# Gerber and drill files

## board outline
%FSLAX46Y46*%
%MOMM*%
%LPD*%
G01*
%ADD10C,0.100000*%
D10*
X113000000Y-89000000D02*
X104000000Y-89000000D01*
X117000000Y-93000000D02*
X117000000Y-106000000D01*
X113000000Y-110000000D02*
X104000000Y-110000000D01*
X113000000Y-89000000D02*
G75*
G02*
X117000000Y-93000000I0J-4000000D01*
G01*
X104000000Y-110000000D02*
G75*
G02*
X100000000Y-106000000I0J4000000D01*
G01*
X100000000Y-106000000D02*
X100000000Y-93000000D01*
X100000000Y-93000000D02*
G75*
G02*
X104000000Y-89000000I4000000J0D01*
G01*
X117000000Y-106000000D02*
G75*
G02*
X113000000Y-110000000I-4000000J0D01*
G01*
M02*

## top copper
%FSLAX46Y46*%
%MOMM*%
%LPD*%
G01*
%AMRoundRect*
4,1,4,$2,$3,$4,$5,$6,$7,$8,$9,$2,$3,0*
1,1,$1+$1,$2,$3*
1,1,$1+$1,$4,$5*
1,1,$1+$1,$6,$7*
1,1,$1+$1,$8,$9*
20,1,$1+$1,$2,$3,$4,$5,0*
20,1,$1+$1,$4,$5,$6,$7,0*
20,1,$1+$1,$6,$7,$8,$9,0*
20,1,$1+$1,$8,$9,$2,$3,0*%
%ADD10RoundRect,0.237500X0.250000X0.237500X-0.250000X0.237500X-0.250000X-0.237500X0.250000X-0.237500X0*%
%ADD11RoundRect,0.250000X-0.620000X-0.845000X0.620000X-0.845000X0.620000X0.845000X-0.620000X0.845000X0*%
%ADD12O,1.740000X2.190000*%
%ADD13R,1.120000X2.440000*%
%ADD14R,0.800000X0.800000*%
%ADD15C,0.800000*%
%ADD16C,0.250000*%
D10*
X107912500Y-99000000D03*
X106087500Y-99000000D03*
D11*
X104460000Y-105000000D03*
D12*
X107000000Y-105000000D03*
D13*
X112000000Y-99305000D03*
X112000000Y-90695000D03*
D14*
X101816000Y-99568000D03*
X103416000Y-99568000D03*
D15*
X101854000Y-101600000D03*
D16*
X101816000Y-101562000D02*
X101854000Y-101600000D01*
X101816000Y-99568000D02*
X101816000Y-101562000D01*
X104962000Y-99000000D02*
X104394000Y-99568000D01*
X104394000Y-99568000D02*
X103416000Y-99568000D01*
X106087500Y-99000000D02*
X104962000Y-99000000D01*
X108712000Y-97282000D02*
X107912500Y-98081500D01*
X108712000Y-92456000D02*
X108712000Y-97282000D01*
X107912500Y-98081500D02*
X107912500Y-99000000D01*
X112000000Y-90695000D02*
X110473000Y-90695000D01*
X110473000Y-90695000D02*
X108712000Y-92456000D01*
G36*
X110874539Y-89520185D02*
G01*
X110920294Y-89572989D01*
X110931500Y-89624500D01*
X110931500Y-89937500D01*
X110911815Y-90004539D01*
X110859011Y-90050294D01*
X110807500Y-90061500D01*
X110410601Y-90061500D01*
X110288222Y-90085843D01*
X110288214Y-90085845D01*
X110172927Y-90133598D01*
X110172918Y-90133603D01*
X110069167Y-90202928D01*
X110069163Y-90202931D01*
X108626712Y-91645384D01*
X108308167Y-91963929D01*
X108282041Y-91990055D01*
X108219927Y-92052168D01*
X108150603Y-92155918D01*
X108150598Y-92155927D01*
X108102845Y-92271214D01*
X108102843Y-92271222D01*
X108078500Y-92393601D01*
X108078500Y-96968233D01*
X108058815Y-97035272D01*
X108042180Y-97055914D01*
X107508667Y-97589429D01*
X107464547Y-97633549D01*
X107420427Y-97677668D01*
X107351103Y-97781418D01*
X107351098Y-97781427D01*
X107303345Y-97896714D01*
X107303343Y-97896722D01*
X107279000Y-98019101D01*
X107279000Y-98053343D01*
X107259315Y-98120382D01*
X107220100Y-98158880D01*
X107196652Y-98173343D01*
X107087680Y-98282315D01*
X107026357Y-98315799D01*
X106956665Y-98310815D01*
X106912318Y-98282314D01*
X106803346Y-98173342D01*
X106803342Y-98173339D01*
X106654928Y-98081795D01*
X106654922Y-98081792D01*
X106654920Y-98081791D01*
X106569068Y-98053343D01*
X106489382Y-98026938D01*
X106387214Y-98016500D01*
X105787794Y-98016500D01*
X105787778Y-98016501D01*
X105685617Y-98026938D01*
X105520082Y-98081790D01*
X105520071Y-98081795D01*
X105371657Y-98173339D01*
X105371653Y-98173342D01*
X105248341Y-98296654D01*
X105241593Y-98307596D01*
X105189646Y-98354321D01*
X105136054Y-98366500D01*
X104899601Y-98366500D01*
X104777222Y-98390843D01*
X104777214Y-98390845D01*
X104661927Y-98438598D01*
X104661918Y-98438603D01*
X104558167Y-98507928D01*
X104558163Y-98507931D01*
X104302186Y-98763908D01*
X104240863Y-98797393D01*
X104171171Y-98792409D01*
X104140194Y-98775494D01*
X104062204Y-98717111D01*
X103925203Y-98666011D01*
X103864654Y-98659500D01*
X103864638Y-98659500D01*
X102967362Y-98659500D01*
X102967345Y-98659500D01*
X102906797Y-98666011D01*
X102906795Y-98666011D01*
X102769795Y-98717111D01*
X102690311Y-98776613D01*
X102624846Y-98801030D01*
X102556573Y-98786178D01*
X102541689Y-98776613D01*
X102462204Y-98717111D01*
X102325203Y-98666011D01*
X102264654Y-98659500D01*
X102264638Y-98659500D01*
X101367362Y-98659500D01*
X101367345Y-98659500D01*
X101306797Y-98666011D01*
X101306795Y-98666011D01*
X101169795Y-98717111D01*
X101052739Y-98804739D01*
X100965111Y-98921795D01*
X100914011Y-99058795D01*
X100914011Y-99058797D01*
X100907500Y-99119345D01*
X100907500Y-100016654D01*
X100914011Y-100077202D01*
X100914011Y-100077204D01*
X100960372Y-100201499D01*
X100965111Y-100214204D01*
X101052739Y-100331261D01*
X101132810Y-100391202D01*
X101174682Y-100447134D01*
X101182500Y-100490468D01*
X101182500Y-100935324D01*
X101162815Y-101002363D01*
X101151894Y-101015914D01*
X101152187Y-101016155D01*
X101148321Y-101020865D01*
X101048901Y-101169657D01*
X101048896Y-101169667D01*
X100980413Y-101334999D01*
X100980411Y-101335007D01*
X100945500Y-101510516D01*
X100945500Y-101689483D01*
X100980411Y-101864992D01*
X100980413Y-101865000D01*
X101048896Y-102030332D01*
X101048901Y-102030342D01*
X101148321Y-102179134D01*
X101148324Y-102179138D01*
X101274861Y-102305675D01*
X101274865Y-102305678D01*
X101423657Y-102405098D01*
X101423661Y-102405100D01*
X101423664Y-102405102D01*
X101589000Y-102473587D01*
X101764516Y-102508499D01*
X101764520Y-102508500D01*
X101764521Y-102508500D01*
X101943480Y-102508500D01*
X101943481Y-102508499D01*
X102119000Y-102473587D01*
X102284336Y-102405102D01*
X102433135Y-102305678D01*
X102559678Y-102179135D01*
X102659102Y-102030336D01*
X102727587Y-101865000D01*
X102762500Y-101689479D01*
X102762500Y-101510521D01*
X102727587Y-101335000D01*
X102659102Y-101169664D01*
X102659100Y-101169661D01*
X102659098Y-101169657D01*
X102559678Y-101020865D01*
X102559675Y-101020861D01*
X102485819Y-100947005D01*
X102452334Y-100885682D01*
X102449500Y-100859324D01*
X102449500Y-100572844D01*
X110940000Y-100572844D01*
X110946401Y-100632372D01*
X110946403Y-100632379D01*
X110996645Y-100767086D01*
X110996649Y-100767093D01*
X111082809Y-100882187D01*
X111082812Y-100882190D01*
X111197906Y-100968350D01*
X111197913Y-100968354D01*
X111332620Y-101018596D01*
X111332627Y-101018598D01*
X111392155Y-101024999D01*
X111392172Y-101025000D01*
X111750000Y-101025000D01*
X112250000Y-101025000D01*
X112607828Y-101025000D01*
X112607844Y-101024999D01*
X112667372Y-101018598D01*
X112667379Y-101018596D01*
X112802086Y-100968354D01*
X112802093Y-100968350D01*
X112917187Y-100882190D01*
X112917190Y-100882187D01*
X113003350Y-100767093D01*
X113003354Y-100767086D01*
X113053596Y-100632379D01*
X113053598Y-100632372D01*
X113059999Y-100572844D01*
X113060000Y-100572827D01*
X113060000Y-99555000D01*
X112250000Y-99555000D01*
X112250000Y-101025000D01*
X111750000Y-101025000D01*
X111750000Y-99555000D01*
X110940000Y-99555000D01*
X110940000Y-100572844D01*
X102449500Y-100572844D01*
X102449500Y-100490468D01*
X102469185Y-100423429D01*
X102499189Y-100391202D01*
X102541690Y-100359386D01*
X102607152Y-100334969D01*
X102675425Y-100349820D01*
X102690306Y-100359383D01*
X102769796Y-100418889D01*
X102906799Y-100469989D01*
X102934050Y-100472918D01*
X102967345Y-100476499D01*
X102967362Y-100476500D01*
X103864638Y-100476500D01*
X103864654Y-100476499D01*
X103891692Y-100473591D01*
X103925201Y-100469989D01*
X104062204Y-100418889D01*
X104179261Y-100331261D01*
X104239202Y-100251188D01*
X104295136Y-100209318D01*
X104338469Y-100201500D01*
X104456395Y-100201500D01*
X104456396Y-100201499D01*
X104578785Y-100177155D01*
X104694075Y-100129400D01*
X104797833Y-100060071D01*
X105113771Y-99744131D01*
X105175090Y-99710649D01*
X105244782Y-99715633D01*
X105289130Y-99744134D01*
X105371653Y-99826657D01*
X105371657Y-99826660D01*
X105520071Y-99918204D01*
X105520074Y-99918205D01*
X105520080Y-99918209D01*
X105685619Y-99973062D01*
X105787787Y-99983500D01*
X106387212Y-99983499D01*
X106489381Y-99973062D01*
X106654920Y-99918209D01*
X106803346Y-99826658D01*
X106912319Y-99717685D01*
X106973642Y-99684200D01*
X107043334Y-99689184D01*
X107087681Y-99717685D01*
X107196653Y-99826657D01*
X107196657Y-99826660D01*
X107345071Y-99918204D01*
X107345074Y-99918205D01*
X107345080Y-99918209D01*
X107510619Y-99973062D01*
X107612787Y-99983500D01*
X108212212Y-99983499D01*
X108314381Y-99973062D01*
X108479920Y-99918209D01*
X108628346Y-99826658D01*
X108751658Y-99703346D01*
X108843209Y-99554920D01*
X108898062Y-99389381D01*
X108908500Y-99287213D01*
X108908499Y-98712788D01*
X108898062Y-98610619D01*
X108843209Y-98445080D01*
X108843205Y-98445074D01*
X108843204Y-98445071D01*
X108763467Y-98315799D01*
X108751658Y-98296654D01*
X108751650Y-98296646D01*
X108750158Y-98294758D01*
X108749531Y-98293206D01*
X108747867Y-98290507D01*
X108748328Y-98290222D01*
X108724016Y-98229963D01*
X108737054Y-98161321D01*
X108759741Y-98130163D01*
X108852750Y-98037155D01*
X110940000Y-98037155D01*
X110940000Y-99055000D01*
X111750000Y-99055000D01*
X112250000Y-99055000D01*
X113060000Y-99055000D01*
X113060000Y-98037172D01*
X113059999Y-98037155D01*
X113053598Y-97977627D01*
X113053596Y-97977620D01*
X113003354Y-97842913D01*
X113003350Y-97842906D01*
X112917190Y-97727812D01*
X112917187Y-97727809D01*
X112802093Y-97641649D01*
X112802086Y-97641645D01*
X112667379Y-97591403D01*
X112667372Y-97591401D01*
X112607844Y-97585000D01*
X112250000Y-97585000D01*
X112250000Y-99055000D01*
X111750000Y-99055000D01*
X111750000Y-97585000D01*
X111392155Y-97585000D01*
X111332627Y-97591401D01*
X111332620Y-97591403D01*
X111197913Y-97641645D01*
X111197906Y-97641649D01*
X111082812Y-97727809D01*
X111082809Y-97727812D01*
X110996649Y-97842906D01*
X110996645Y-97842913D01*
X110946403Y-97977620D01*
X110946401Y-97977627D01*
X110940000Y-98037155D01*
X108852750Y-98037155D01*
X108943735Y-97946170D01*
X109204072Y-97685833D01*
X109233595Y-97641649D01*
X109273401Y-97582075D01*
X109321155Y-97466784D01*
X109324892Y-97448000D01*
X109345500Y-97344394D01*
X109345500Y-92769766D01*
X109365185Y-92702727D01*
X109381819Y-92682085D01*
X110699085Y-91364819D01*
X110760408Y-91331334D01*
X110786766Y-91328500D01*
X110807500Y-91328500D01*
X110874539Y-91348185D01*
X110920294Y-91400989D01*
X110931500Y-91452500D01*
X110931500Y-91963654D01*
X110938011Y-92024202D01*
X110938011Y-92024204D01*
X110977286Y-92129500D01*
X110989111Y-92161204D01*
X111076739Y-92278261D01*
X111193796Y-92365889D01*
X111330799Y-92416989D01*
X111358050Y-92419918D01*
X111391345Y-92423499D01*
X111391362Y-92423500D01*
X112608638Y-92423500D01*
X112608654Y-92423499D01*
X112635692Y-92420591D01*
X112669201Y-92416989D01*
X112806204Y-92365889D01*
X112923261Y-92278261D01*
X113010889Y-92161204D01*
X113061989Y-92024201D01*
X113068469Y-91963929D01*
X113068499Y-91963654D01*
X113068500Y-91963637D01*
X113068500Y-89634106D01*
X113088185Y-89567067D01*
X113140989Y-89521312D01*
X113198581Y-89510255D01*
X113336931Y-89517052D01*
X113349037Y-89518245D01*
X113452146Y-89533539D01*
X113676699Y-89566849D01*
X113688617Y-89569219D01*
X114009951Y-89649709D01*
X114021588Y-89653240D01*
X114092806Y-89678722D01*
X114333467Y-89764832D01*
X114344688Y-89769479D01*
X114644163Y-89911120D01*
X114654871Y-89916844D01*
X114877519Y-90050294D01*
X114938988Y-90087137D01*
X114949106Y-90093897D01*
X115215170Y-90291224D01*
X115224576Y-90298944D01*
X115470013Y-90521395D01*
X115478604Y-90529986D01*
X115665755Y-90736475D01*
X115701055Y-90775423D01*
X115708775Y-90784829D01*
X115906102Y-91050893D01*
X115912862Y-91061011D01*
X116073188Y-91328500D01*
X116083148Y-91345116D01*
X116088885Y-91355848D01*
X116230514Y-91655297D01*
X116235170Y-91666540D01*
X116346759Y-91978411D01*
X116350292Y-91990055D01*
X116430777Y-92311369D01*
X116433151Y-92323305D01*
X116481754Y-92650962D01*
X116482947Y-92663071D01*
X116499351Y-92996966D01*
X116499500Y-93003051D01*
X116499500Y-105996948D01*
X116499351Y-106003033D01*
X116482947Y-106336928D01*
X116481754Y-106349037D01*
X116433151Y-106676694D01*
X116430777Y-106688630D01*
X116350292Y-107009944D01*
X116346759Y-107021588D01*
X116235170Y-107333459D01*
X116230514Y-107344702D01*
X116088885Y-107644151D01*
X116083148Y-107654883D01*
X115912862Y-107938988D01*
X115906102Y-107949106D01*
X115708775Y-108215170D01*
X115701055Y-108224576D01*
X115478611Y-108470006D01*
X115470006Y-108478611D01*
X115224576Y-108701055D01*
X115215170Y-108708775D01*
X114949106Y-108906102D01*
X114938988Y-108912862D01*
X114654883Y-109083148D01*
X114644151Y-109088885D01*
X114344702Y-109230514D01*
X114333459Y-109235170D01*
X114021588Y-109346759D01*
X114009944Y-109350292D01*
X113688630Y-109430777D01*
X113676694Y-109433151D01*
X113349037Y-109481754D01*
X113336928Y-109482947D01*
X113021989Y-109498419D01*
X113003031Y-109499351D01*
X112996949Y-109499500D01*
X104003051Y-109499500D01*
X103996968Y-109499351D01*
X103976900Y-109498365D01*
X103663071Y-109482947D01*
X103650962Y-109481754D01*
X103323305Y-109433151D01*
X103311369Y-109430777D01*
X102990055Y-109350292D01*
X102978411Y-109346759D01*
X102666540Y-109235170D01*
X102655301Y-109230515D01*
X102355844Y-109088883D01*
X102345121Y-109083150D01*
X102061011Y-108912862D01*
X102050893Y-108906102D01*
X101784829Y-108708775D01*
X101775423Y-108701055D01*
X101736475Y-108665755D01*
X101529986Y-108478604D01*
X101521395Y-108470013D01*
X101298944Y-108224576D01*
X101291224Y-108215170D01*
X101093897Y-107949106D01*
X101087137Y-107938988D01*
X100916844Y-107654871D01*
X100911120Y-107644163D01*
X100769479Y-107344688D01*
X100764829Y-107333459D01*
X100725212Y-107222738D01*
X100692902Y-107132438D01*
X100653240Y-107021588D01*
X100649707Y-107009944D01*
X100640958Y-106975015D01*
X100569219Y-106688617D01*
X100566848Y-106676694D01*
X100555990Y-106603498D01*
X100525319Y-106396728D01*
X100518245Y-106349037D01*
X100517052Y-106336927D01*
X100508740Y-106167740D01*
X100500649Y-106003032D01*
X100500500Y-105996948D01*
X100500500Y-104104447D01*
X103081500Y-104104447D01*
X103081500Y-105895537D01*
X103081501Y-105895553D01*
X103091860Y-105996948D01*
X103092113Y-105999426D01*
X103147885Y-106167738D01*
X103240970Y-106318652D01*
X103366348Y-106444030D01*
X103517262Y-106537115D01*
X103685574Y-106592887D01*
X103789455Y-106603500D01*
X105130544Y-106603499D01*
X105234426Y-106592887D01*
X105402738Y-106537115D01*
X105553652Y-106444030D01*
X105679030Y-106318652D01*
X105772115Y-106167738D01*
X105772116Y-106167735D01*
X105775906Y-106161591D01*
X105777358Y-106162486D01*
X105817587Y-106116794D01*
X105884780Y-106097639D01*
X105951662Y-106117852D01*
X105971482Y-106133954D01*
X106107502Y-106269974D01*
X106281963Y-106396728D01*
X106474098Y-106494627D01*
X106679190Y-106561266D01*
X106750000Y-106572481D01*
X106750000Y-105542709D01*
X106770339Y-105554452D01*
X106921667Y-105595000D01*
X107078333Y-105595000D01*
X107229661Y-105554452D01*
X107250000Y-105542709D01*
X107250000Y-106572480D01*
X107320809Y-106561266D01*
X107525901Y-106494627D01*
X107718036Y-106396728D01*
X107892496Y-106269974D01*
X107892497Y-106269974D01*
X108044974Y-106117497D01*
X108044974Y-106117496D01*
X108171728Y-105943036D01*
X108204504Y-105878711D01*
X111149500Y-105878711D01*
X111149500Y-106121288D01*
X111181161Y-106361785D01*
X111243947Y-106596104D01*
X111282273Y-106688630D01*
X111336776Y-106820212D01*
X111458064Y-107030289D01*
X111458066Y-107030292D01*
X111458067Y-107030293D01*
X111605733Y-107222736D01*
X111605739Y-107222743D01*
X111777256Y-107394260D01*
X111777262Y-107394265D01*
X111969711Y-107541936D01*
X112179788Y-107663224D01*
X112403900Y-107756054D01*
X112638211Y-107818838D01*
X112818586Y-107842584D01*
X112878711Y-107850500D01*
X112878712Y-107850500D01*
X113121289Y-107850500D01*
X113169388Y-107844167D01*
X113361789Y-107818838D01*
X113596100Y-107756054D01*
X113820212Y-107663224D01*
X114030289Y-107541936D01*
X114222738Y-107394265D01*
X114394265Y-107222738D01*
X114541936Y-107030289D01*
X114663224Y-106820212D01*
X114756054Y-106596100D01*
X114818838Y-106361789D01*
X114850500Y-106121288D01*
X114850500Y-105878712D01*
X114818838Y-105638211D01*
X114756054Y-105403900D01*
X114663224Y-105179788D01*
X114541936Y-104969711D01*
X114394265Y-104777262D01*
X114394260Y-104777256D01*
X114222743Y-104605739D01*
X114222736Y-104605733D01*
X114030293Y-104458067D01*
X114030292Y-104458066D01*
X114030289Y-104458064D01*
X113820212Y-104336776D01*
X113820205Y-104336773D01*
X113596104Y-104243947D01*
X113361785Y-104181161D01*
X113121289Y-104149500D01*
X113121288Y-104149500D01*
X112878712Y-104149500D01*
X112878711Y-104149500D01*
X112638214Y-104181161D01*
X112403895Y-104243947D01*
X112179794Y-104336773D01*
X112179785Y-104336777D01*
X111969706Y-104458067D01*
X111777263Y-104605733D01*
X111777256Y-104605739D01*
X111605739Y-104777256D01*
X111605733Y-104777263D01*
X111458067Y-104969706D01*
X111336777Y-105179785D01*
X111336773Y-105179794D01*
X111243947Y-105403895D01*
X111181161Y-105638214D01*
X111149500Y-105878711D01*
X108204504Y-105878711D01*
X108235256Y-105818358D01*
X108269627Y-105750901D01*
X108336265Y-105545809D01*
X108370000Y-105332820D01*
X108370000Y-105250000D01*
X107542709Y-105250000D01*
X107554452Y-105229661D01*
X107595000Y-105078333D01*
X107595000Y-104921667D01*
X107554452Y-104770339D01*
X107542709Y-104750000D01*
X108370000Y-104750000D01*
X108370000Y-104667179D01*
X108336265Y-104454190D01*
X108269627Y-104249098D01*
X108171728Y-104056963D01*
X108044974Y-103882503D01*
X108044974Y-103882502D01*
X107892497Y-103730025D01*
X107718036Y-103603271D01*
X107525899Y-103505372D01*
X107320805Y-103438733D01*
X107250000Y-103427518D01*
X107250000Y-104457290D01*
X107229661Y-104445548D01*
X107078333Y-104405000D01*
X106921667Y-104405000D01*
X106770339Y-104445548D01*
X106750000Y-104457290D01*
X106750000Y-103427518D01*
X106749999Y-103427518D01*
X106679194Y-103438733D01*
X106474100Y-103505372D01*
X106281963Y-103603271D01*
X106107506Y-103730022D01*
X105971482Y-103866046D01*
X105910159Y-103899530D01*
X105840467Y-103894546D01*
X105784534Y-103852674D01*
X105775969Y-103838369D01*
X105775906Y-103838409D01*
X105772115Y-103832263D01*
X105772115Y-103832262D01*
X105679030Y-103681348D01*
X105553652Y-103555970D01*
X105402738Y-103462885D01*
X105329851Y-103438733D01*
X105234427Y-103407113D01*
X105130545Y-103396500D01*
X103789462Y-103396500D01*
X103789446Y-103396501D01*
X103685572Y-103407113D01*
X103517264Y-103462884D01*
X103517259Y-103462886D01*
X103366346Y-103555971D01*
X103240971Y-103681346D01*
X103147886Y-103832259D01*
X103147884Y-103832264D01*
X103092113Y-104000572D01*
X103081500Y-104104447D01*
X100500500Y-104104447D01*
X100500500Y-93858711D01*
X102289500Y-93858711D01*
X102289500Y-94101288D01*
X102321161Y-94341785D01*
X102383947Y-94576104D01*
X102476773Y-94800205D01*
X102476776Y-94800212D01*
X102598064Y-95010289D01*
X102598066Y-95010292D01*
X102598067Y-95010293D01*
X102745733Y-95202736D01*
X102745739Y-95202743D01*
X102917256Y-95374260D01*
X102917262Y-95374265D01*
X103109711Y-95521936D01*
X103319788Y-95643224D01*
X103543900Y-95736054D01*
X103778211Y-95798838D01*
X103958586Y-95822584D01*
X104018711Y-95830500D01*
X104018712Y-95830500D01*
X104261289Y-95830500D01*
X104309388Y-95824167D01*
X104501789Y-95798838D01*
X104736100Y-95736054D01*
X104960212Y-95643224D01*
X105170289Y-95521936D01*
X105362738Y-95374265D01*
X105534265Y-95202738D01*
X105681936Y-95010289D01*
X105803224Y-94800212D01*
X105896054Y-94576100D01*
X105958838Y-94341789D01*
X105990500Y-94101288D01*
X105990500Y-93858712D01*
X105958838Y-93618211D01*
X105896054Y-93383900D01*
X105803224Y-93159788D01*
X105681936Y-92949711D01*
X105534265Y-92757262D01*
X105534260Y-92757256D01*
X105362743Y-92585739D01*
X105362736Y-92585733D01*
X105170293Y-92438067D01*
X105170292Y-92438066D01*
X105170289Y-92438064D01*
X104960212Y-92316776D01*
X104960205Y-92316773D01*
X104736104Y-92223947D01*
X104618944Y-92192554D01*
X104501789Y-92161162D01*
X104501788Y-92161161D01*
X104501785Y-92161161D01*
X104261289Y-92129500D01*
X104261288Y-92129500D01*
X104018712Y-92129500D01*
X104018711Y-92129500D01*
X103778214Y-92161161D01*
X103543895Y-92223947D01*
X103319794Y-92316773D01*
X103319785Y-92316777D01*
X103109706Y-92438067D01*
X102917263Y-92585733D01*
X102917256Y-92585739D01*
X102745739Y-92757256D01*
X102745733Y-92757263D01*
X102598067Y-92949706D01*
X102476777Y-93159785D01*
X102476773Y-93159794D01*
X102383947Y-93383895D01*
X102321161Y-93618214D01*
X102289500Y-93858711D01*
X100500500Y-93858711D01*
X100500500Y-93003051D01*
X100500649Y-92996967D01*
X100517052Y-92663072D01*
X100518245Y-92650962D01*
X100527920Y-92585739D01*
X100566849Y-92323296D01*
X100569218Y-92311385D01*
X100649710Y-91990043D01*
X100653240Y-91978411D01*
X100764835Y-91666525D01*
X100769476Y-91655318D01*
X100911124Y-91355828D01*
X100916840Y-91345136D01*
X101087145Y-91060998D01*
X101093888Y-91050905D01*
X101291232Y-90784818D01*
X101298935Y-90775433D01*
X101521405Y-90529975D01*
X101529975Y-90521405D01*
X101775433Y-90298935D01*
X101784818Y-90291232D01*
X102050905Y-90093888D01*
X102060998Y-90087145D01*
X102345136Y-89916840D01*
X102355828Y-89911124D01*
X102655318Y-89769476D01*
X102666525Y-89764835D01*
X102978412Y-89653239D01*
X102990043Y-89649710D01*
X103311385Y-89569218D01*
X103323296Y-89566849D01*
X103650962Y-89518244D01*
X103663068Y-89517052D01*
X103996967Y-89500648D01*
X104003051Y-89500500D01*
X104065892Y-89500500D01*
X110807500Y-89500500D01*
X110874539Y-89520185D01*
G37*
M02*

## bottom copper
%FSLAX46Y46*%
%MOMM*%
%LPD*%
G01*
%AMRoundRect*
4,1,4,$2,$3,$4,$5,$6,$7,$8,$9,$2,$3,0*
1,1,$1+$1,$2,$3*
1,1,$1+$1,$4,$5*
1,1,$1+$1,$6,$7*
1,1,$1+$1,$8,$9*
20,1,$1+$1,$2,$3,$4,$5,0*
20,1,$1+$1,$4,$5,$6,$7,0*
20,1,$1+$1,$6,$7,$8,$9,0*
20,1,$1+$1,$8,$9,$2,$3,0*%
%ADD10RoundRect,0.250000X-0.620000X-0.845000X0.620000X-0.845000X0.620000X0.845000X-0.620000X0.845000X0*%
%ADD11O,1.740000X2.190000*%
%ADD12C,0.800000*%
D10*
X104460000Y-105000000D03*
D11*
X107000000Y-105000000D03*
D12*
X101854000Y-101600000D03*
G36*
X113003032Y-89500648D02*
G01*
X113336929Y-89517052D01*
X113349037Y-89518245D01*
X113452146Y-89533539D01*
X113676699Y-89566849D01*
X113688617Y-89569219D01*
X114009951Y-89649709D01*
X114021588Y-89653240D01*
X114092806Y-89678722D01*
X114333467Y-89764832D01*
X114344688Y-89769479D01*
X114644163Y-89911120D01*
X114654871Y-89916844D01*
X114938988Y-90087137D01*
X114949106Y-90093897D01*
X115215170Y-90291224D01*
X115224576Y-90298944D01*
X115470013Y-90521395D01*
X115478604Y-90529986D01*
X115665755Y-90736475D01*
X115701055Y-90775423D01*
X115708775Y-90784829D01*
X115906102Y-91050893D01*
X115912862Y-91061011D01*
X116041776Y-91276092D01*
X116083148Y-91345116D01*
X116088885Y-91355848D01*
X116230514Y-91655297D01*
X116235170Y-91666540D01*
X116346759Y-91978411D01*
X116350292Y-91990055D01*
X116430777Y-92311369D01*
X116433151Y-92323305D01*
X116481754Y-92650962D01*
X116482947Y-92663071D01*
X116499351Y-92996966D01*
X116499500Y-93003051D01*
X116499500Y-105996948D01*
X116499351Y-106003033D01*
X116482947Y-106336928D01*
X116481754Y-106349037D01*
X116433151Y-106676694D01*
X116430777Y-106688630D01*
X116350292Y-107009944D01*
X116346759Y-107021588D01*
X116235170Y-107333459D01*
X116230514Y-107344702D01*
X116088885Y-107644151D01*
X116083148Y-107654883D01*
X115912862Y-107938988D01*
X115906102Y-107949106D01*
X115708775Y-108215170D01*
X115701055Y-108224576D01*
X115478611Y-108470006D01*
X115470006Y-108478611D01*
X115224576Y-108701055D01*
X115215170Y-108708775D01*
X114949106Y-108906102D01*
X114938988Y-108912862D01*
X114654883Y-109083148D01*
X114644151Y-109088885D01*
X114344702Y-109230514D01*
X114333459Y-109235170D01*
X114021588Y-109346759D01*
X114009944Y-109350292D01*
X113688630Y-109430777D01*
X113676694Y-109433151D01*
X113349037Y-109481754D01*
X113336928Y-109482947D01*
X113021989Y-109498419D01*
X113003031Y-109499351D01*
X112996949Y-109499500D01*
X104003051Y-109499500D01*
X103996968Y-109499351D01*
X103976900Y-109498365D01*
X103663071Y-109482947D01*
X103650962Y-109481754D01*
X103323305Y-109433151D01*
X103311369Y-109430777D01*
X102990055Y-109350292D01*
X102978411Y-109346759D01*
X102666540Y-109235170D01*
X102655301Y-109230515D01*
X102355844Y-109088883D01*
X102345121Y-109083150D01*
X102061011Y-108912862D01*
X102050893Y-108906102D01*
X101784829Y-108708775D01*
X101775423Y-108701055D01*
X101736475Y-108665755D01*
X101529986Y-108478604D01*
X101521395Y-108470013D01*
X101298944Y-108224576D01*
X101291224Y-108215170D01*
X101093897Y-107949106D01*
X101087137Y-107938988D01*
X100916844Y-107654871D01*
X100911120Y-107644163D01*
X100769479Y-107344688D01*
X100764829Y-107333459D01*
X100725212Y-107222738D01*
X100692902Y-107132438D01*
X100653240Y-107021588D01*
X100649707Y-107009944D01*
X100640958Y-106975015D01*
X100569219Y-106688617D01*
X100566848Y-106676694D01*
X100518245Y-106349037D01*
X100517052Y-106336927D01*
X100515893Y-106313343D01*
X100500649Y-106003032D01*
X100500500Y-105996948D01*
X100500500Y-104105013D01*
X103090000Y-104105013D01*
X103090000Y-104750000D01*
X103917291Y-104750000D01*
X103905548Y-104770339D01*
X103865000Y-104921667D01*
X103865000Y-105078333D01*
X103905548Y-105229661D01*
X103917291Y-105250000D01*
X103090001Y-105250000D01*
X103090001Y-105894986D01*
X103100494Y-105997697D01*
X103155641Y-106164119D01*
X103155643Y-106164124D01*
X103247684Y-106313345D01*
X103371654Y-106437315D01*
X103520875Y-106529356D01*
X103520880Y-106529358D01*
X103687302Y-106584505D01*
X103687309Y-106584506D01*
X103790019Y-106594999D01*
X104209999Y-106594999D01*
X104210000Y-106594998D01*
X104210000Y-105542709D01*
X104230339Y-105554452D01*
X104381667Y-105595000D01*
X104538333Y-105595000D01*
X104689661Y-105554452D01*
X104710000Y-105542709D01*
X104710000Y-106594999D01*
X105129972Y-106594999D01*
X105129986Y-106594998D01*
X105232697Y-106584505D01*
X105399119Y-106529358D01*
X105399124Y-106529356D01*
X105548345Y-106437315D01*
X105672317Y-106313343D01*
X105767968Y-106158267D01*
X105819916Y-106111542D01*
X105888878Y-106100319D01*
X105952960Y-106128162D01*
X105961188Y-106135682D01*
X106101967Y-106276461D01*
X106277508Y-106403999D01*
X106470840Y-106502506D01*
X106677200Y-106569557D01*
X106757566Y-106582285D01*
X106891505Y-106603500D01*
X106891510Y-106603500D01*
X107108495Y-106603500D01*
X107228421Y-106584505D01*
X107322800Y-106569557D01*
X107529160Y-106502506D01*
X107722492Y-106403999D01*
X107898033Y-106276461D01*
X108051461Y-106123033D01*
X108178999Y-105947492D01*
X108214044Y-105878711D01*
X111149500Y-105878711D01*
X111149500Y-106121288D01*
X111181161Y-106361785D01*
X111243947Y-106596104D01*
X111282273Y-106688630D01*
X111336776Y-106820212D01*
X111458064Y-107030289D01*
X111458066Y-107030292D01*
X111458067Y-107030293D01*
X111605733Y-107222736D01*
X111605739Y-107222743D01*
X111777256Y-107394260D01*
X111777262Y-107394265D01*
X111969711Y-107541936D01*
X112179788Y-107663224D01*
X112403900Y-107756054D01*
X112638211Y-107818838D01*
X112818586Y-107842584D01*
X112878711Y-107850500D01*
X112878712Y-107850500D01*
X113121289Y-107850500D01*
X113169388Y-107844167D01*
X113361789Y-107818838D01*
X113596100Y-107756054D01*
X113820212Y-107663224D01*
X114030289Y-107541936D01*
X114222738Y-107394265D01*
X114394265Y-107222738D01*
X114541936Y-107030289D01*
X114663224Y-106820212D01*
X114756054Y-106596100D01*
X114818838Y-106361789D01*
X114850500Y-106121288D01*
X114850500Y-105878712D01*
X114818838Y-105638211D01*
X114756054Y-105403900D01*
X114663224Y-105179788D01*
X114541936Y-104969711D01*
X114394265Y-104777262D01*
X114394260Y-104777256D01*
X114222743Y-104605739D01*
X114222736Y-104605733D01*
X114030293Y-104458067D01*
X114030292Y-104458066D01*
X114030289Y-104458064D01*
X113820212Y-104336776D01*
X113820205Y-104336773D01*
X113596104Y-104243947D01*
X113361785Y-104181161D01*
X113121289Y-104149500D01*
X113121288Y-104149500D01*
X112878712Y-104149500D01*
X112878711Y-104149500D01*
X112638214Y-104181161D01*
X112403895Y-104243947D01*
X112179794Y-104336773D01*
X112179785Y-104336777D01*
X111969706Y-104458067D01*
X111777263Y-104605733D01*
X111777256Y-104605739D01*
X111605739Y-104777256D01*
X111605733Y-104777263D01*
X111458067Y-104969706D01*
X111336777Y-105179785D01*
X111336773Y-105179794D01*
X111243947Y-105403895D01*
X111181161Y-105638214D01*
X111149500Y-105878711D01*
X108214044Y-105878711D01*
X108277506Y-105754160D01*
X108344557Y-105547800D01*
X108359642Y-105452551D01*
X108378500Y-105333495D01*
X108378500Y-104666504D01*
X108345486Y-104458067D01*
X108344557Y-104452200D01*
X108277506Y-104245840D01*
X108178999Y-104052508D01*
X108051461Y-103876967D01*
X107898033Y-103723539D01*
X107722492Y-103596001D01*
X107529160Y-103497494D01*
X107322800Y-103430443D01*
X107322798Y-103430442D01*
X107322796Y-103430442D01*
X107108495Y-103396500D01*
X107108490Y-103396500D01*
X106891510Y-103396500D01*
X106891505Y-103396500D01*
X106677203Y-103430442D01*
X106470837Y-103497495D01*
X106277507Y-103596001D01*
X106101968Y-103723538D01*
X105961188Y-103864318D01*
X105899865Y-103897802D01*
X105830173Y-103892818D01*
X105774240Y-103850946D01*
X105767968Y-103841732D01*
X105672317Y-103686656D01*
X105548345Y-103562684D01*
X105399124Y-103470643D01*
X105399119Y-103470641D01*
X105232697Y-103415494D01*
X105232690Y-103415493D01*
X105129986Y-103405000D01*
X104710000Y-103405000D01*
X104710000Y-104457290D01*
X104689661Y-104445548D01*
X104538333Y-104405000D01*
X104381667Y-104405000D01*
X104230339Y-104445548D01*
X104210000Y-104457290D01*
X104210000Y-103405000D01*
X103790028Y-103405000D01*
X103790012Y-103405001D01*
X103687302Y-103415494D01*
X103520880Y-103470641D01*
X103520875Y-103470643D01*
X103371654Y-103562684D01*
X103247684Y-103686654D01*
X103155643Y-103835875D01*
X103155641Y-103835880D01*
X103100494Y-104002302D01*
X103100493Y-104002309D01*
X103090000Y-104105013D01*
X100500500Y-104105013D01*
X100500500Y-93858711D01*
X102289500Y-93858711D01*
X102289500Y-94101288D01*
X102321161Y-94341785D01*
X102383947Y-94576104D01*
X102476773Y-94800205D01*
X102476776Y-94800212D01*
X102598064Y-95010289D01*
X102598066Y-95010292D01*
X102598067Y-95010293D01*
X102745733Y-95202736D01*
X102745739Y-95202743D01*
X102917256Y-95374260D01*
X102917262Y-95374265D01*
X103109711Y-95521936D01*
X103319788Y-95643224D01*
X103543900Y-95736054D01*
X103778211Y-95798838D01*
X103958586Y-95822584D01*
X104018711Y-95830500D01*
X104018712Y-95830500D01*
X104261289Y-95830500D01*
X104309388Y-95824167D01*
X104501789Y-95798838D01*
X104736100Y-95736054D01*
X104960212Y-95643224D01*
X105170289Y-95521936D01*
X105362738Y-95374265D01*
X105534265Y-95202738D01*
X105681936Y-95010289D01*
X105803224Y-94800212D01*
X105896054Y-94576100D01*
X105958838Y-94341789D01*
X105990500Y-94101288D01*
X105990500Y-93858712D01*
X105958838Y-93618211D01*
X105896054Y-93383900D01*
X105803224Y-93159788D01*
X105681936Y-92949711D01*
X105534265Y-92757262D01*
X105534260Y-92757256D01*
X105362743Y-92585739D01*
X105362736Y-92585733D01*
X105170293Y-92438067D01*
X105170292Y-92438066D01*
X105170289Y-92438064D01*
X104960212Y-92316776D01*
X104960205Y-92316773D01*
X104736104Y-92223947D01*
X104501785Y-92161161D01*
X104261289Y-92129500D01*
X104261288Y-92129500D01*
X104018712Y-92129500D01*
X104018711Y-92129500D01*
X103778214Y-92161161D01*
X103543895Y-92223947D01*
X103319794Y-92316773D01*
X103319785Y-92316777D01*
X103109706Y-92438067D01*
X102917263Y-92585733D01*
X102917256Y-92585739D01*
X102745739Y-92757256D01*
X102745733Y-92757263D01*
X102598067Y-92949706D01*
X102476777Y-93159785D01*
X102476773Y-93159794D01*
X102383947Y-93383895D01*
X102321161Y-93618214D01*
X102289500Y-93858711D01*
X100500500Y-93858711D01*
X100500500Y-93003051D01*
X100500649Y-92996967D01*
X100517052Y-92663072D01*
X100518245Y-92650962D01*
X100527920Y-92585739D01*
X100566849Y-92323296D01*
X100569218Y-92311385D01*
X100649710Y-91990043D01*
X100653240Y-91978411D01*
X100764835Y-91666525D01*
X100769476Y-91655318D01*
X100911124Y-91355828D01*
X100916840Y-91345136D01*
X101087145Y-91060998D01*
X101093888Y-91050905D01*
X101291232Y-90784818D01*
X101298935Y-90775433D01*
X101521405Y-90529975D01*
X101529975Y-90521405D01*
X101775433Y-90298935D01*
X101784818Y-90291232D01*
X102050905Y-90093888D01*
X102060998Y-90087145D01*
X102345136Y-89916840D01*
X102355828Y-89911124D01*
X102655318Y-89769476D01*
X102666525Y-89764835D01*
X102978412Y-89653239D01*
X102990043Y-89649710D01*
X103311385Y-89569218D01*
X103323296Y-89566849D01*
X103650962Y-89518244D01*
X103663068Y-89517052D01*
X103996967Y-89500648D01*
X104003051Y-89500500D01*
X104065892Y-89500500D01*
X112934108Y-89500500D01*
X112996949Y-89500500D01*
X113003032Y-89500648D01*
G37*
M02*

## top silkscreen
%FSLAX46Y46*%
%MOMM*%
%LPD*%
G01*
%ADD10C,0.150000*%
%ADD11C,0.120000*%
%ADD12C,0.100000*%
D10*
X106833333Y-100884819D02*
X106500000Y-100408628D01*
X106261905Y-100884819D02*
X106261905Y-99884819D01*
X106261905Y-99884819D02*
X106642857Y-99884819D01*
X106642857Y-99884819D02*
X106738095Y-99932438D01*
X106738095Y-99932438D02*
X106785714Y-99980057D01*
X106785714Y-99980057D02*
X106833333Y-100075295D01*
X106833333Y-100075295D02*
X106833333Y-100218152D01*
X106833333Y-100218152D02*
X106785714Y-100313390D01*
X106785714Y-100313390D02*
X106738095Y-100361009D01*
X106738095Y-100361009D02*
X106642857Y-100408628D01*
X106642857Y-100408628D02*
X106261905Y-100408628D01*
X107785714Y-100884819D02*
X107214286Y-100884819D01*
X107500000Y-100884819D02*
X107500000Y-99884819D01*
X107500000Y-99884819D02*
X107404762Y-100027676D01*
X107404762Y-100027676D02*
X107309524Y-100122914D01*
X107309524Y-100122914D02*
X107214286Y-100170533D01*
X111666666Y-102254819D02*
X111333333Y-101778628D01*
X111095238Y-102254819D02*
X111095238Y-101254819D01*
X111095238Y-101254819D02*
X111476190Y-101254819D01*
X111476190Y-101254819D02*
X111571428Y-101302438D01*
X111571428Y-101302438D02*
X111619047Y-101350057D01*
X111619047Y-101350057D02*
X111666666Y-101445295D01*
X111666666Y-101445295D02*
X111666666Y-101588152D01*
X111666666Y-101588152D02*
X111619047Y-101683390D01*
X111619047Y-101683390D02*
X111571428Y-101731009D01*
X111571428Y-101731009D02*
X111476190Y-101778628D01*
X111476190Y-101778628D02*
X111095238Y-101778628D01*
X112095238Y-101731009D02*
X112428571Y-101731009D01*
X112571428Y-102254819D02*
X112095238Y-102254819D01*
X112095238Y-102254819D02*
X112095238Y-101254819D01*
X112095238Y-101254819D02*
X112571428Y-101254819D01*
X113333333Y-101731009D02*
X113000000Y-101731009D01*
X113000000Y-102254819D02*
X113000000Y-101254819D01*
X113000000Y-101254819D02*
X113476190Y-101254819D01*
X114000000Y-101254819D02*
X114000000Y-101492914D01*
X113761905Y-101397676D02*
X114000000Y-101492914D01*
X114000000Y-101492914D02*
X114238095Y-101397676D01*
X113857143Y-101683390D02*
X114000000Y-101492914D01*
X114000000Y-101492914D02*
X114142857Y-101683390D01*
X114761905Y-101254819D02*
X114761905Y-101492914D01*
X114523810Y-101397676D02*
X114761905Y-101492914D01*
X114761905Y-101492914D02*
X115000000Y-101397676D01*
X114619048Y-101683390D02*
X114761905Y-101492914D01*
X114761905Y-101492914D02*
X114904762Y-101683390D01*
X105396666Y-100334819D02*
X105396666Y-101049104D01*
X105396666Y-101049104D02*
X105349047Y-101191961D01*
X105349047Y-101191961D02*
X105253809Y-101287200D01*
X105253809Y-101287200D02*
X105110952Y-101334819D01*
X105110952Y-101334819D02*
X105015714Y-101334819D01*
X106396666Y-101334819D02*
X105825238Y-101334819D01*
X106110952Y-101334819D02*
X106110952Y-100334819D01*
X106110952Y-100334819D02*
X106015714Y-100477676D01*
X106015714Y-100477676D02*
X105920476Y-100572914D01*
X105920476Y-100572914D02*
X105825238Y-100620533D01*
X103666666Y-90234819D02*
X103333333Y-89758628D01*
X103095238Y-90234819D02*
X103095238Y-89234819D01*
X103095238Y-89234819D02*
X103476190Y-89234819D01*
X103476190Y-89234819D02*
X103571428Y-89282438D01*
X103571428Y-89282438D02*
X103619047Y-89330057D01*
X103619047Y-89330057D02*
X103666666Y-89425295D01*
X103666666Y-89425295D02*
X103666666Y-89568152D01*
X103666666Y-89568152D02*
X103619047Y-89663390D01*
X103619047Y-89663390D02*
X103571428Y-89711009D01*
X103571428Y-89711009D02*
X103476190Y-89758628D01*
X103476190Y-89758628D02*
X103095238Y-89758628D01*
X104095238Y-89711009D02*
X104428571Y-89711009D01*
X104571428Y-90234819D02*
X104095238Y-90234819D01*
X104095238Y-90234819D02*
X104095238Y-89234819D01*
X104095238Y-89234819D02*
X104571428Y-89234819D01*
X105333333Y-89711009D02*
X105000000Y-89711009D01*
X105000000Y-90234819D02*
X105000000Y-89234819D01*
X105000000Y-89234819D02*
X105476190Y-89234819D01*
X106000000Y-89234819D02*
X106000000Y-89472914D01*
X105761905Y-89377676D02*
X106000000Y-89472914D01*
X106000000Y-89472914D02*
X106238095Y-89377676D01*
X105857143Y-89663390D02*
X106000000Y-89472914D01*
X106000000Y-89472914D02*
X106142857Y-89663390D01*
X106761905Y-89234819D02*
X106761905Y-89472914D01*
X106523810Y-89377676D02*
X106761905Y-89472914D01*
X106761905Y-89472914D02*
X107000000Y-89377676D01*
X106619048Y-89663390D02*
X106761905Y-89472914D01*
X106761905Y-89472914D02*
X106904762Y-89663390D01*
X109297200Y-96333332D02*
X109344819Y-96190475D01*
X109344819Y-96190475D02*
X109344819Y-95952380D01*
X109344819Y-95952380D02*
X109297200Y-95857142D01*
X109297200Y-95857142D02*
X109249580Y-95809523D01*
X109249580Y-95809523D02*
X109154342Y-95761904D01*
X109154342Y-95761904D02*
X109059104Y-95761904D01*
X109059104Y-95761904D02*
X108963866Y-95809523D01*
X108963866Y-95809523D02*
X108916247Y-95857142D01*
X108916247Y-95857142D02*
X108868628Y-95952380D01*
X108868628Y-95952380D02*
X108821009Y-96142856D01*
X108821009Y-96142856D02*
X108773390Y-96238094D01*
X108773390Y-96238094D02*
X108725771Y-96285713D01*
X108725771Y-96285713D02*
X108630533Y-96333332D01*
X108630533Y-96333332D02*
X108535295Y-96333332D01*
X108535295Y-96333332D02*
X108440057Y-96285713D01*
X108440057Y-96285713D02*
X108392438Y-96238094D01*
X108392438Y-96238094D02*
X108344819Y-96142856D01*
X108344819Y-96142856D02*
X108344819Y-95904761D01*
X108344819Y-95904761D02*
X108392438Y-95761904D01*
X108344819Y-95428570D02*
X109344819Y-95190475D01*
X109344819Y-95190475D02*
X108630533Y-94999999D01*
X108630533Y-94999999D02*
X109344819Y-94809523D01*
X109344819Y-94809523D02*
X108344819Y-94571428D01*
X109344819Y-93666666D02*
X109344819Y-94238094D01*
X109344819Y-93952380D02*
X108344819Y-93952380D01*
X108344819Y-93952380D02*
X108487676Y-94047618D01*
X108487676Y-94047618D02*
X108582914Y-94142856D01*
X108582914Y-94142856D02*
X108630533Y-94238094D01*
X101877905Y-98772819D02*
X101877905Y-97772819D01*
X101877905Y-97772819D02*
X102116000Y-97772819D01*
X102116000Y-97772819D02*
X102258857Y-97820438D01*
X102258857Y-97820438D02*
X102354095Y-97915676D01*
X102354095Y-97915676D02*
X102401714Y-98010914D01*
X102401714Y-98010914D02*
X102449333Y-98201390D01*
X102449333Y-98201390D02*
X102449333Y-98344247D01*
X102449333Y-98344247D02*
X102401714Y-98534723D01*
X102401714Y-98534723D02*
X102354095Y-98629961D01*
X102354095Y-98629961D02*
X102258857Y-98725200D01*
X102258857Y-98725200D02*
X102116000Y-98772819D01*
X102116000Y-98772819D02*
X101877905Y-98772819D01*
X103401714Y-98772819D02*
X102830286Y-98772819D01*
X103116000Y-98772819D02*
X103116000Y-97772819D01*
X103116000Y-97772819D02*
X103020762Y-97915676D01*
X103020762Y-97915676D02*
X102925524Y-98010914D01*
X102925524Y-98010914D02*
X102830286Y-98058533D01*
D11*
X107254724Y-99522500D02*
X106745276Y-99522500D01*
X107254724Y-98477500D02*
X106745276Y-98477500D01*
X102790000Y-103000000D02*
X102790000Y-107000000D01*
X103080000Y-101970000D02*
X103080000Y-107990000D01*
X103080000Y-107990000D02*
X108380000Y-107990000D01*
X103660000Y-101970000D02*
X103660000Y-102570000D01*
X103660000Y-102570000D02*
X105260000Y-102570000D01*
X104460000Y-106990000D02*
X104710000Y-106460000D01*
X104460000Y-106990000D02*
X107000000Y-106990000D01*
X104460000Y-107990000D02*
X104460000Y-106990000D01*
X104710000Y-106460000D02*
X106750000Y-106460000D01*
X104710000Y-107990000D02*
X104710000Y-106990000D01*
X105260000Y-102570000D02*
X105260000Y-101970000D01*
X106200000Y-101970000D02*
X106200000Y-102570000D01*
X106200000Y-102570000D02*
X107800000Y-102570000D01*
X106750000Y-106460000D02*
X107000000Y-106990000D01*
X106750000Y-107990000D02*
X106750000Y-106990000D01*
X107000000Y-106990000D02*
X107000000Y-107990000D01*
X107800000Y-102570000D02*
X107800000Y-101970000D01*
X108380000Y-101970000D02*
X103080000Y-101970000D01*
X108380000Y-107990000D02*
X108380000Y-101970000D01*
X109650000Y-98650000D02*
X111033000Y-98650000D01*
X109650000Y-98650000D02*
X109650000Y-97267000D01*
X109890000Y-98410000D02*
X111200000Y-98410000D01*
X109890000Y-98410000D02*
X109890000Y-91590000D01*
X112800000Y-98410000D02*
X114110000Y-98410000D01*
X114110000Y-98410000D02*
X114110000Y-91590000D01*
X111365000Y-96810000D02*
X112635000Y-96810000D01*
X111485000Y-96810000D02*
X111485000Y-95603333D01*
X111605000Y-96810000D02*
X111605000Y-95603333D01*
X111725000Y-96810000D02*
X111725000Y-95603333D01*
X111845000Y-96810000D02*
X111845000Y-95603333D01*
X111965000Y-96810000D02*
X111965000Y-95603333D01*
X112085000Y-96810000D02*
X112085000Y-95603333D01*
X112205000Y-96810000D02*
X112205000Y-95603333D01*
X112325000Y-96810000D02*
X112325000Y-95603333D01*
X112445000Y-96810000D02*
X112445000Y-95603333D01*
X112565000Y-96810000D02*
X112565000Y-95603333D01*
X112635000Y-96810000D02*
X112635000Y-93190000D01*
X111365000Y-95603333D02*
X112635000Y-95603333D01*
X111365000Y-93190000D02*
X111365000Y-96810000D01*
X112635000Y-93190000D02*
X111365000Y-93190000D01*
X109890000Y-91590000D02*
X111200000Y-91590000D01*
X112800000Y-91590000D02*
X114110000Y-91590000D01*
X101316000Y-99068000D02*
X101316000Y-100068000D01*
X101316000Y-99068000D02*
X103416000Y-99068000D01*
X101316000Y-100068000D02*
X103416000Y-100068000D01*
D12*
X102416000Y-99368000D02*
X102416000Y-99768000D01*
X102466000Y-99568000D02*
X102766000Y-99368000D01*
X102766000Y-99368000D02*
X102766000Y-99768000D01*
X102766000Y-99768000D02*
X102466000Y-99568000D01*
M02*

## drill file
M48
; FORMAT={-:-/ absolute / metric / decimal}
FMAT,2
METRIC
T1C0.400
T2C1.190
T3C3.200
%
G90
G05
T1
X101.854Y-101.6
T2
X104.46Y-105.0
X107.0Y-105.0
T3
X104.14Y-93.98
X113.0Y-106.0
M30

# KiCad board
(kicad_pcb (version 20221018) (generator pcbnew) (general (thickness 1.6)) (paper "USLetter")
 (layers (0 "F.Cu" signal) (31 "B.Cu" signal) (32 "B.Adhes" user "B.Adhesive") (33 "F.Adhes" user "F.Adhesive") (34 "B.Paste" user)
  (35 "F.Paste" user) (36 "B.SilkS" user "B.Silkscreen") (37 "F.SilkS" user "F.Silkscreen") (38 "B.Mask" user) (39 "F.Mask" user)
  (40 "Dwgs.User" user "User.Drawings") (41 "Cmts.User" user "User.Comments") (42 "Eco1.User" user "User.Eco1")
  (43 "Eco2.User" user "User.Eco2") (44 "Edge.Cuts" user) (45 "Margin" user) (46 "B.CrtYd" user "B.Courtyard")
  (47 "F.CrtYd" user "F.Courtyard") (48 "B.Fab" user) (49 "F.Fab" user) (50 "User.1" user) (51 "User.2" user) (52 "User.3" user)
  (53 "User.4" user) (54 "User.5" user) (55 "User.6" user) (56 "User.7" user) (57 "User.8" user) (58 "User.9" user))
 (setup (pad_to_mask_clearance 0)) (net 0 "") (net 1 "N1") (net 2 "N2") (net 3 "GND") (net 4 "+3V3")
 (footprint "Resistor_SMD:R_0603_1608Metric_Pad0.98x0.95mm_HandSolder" (layer "F.Cu") (at 107 99 180)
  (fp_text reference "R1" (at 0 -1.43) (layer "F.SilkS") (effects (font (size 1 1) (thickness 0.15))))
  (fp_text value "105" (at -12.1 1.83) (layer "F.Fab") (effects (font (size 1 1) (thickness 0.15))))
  (fp_line (start -0.254724 -0.5225) (end 0.254724 -0.5225) (stroke (width 0.12) (type solid)) (layer "F.SilkS"))
  (fp_line (start -0.254724 0.5225) (end 0.254724 0.5225) (stroke (width 0.12) (type solid)) (layer "F.SilkS"))
  (pad "1" smd roundrect (at -0.9125 0 180) (size 0.975 0.95) (layers "F.Cu" "F.Paste" "F.Mask") (roundrect_rratio 0.25) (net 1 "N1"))
  (pad "2" smd roundrect (at 0.9125 0 180) (size 0.975 0.95) (layers "F.Cu" "F.Paste" "F.Mask") (roundrect_rratio 0.25) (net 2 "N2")))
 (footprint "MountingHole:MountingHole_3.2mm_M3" (layer "F.Cu") (at 113 106)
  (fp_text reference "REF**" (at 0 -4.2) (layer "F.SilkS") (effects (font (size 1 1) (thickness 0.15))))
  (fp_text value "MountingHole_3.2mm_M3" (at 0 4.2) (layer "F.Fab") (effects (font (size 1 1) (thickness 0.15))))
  (pad "" np_thru_hole circle (at 0 0) (size 3.2 3.2) (drill 3.2) (layers "F&B.Cu" "*.Mask")))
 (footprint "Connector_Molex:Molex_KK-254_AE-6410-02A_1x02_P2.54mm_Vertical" (layer "F.Cu") (at 104.46 105)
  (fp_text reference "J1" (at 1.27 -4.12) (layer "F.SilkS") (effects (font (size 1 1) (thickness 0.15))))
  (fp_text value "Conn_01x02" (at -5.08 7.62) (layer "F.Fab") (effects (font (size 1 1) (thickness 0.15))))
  (fp_line (start -1.67 -2) (end -1.67 2) (stroke (width 0.12) (type solid)) (layer "F.SilkS"))
  (fp_line (start -1.38 -3.03) (end -1.38 2.99) (stroke (width 0.12) (type solid)) (layer "F.SilkS"))
  (fp_line (start -1.38 2.99) (end 3.92 2.99) (stroke (width 0.12) (type solid)) (layer "F.SilkS"))
  (fp_line (start -0.8 -3.03) (end -0.8 -2.43) (stroke (width 0.12) (type solid)) (layer "F.SilkS"))
  (fp_line (start -0.8 -2.43) (end 0.8 -2.43) (stroke (width 0.12) (type solid)) (layer "F.SilkS"))
  (fp_line (start 0 1.99) (end 0.25 1.46) (stroke (width 0.12) (type solid)) (layer "F.SilkS"))
  (fp_line (start 0 1.99) (end 2.54 1.99) (stroke (width 0.12) (type solid)) (layer "F.SilkS"))
  (fp_line (start 0 2.99) (end 0 1.99) (stroke (width 0.12) (type solid)) (layer "F.SilkS"))
  (fp_line (start 0.25 1.46) (end 2.29 1.46) (stroke (width 0.12) (type solid)) (layer "F.SilkS"))
  (fp_line (start 0.25 2.99) (end 0.25 1.99) (stroke (width 0.12) (type solid)) (layer "F.SilkS"))
  (fp_line (start 0.8 -2.43) (end 0.8 -3.03) (stroke (width 0.12) (type solid)) (layer "F.SilkS"))
  (fp_line (start 1.74 -3.03) (end 1.74 -2.43) (stroke (width 0.12) (type solid)) (layer "F.SilkS"))
  (fp_line (start 1.74 -2.43) (end 3.34 -2.43) (stroke (width 0.12) (type solid)) (layer "F.SilkS"))
  (fp_line (start 2.29 1.46) (end 2.54 1.99) (stroke (width 0.12) (type solid)) (layer "F.SilkS"))
  (fp_line (start 2.29 2.99) (end 2.29 1.99) (stroke (width 0.12) (type solid)) (layer "F.SilkS"))
  (fp_line (start 2.54 1.99) (end 2.54 2.99) (stroke (width 0.12) (type solid)) (layer "F.SilkS"))
  (fp_line (start 3.34 -2.43) (end 3.34 -3.03) (stroke (width 0.12) (type solid)) (layer "F.SilkS"))
  (fp_line (start 3.92 -3.03) (end -1.38 -3.03) (stroke (width 0.12) (type solid)) (layer "F.SilkS"))
  (fp_line (start 3.92 2.99) (end 3.92 -3.03) (stroke (width 0.12) (type solid)) (layer "F.SilkS"))
  (pad "1" thru_hole roundrect (at 0 0) (size 1.74 2.19) (drill 1.19) (layers "*.Cu" "*.Mask") (roundrect_rratio 0.143678) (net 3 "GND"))
  (pad "2" thru_hole oval (at 2.54 0) (size 1.74 2.19) (drill 1.19) (layers "*.Cu" "*.Mask") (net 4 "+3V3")))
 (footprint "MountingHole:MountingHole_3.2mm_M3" (layer "F.Cu") (at 104.14 93.98)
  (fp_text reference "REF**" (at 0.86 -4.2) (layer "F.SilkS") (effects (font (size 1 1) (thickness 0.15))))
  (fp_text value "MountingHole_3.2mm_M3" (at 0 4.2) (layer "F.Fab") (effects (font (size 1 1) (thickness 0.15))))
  (pad "" np_thru_hole circle (at 0 0) (size 3.2 3.2) (drill 3.2) (layers "*.Cu" "*.Mask")))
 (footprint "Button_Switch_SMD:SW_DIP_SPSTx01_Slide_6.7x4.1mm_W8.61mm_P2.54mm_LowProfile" (layer "F.Cu") (at 112 95 90)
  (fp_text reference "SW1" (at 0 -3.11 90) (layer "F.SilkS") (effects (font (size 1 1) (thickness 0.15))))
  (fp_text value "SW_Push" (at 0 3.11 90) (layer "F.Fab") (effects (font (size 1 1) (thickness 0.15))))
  (fp_line (start -3.65 -2.35) (end -3.65 -0.967) (stroke (width 0.12) (type solid)) (layer "F.SilkS"))
  (fp_line (start -3.65 -2.35) (end -2.267 -2.35) (stroke (width 0.12) (type solid)) (layer "F.SilkS"))
  (fp_line (start -3.41 -2.11) (end -3.41 -0.8) (stroke (width 0.12) (type solid)) (layer "F.SilkS"))
  (fp_line (start -3.41 -2.11) (end 3.41 -2.11) (stroke (width 0.12) (type solid)) (layer "F.SilkS"))
  (fp_line (start -3.41 0.8) (end -3.41 2.11) (stroke (width 0.12) (type solid)) (layer "F.SilkS"))
  (fp_line (start -3.41 2.11) (end 3.41 2.11) (stroke (width 0.12) (type solid)) (layer "F.SilkS"))
  (fp_line (start -1.81 -0.635) (end -1.81 0.635) (stroke (width 0.12) (type solid)) (layer "F.SilkS"))
  (fp_line (start -1.81 -0.515) (end -0.603333 -0.515) (stroke (width 0.12) (type solid)) (layer "F.SilkS"))
  (fp_line (start -1.81 -0.395) (end -0.603333 -0.395) (stroke (width 0.12) (type solid)) (layer "F.SilkS"))
  (fp_line (start -1.81 -0.275) (end -0.603333 -0.275) (stroke (width 0.12) (type solid)) (layer "F.SilkS"))
  (fp_line (start -1.81 -0.155) (end -0.603333 -0.155) (stroke (width 0.12) (type solid)) (layer "F.SilkS"))
  (fp_line (start -1.81 -0.035) (end -0.603333 -0.035) (stroke (width 0.12) (type solid)) (layer "F.SilkS"))
  (fp_line (start -1.81 0.085) (end -0.603333 0.085) (stroke (width 0.12) (type solid)) (layer "F.SilkS"))
  (fp_line (start -1.81 0.205) (end -0.603333 0.205) (stroke (width 0.12) (type solid)) (layer "F.SilkS"))
  (fp_line (start -1.81 0.325) (end -0.603333 0.325) (stroke (width 0.12) (type solid)) (layer "F.SilkS"))
  (fp_line (start -1.81 0.445) (end -0.603333 0.445) (stroke (width 0.12) (type solid)) (layer "F.SilkS"))
  (fp_line (start -1.81 0.565) (end -0.603333 0.565) (stroke (width 0.12) (type solid)) (layer "F.SilkS"))
  (fp_line (start -1.81 0.635) (end 1.81 0.635) (stroke (width 0.12) (type solid)) (layer "F.SilkS"))
  (fp_line (start -0.603333 -0.635) (end -0.603333 0.635) (stroke (width 0.12) (type solid)) (layer "F.SilkS"))
  (fp_line (start 1.81 -0.635) (end -1.81 -0.635) (stroke (width 0.12) (type solid)) (layer "F.SilkS"))
  (fp_line (start 1.81 0.635) (end 1.81 -0.635) (stroke (width 0.12) (type solid)) (layer "F.SilkS"))
  (fp_line (start 3.41 -2.11) (end 3.41 -0.8) (stroke (width 0.12) (type solid)) (layer "F.SilkS"))
  (fp_line (start 3.41 0.8) (end 3.41 2.11) (stroke (width 0.12) (type solid)) (layer "F.SilkS"))
  (pad "1" smd rect (at -4.305 0 90) (size 2.44 1.12) (layers "F.Cu" "F.Paste" "F.Mask") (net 4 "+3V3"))
  (pad "2" smd rect (at 4.305 0 90) (size 2.44 1.12) (layers "F.Cu" "F.Paste" "F.Mask") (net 1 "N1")))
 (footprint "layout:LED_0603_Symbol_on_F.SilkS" (layer "F.Cu") (at 102.616 99.568)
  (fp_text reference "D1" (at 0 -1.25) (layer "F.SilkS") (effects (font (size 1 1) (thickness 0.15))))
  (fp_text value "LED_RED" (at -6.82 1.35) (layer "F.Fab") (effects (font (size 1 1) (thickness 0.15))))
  (fp_line (start -1.3 -0.5) (end -1.3 0.5) (stroke (width 0.12) (type solid)) (layer "F.SilkS"))
  (fp_line (start -1.3 -0.5) (end 0.8 -0.5) (stroke (width 0.12) (type solid)) (layer "F.SilkS"))
  (fp_line (start -1.3 0.5) (end 0.8 0.5) (stroke (width 0.12) (type solid)) (layer "F.SilkS"))
  (fp_line (start -0.2 -0.2) (end -0.2 0.2) (stroke (width 0.1) (type solid)) (layer "F.SilkS"))
  (fp_line (start -0.15 0) (end 0.15 -0.2) (stroke (width 0.1) (type solid)) (layer "F.SilkS"))
  (fp_line (start 0.15 -0.2) (end 0.15 0.2) (stroke (width 0.1) (type solid)) (layer "F.SilkS"))
  (fp_line (start 0.15 0.2) (end -0.15 0) (stroke (width 0.1) (type solid)) (layer "F.SilkS"))
  (pad "1" smd rect (at -0.8 0 180) (size 0.8 0.8) (layers "F.Cu" "F.Paste" "F.Mask") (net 3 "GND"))
  (pad "2" smd rect (at 0.8 0 180) (size 0.8 0.8) (layers "F.Cu" "F.Paste" "F.Mask") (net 2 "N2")))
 (gr_line (start 113 89) (end 104 89) (stroke (width 0.1) (type default)) (layer "Edge.Cuts"))
 (gr_line (start 117 93) (end 117 106) (stroke (width 0.1) (type default)) (layer "Edge.Cuts"))
 (gr_line (start 113 110) (end 104 110) (stroke (width 0.1) (type default)) (layer "Edge.Cuts"))
 (gr_arc (start 113 89) (mid 115.828427 90.171573) (end 117 93) (stroke (width 0.1) (type default)) (layer "Edge.Cuts"))
 (gr_arc (start 104 110) (mid 101.171573 108.828427) (end 100 106) (stroke (width 0.1) (type default)) (layer "Edge.Cuts"))
 (gr_line (start 100 106) (end 100 93) (stroke (width 0.1) (type default)) (layer "Edge.Cuts"))
 (gr_arc (start 100 93) (mid 101.171573 90.171573) (end 104 89) (stroke (width 0.1) (type default)) (layer "Edge.Cuts"))
 (gr_arc (start 117 106) (mid 115.828427 108.828427) (end 113 110) (stroke (width 0.1) (type default)) (layer "Edge.Cuts"))
 (segment (start 101.816 101.562) (end 101.854 101.6) (width 0.25) (layer "F.Cu") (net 3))
 (segment (start 101.816 99.568) (end 101.816 101.562) (width 0.25) (layer "F.Cu") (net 3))
 (via (at 101.854 101.6) (size 0.8) (drill 0.4) (layers "F.Cu" "B.Cu") (free) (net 3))
 (segment (start 104.962 99) (end 104.394 99.568) (width 0.25) (layer "F.Cu") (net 2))
 (segment (start 104.394 99.568) (end 103.416 99.568) (width 0.25) (layer "F.Cu") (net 2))
 (segment (start 106.0875 99) (end 104.962 99) (width 0.25) (layer "F.Cu") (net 2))
 (segment (start 108.712 97.282) (end 107.9125 98.0815) (width 0.25) (layer "F.Cu") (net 1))
 (segment (start 108.712 92.456) (end 108.712 97.282) (width 0.25) (layer "F.Cu") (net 1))
 (segment (start 107.9125 98.0815) (end 107.9125 99) (width 0.25) (layer "F.Cu") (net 1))
 (segment (start 112 90.695) (end 110.473 90.695) (width 0.25) (layer "F.Cu") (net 1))
 (segment (start 110.473 90.695) (end 108.712 92.456) (width 0.25) (layer "F.Cu") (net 1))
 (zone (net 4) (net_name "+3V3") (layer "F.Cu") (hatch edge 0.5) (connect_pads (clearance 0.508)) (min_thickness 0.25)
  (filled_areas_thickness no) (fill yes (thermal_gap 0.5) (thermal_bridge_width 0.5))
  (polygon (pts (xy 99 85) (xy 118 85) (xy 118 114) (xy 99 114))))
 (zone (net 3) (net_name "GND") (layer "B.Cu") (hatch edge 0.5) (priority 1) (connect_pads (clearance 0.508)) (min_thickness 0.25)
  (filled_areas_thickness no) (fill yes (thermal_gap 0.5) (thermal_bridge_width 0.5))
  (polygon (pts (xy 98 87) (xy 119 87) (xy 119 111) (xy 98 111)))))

